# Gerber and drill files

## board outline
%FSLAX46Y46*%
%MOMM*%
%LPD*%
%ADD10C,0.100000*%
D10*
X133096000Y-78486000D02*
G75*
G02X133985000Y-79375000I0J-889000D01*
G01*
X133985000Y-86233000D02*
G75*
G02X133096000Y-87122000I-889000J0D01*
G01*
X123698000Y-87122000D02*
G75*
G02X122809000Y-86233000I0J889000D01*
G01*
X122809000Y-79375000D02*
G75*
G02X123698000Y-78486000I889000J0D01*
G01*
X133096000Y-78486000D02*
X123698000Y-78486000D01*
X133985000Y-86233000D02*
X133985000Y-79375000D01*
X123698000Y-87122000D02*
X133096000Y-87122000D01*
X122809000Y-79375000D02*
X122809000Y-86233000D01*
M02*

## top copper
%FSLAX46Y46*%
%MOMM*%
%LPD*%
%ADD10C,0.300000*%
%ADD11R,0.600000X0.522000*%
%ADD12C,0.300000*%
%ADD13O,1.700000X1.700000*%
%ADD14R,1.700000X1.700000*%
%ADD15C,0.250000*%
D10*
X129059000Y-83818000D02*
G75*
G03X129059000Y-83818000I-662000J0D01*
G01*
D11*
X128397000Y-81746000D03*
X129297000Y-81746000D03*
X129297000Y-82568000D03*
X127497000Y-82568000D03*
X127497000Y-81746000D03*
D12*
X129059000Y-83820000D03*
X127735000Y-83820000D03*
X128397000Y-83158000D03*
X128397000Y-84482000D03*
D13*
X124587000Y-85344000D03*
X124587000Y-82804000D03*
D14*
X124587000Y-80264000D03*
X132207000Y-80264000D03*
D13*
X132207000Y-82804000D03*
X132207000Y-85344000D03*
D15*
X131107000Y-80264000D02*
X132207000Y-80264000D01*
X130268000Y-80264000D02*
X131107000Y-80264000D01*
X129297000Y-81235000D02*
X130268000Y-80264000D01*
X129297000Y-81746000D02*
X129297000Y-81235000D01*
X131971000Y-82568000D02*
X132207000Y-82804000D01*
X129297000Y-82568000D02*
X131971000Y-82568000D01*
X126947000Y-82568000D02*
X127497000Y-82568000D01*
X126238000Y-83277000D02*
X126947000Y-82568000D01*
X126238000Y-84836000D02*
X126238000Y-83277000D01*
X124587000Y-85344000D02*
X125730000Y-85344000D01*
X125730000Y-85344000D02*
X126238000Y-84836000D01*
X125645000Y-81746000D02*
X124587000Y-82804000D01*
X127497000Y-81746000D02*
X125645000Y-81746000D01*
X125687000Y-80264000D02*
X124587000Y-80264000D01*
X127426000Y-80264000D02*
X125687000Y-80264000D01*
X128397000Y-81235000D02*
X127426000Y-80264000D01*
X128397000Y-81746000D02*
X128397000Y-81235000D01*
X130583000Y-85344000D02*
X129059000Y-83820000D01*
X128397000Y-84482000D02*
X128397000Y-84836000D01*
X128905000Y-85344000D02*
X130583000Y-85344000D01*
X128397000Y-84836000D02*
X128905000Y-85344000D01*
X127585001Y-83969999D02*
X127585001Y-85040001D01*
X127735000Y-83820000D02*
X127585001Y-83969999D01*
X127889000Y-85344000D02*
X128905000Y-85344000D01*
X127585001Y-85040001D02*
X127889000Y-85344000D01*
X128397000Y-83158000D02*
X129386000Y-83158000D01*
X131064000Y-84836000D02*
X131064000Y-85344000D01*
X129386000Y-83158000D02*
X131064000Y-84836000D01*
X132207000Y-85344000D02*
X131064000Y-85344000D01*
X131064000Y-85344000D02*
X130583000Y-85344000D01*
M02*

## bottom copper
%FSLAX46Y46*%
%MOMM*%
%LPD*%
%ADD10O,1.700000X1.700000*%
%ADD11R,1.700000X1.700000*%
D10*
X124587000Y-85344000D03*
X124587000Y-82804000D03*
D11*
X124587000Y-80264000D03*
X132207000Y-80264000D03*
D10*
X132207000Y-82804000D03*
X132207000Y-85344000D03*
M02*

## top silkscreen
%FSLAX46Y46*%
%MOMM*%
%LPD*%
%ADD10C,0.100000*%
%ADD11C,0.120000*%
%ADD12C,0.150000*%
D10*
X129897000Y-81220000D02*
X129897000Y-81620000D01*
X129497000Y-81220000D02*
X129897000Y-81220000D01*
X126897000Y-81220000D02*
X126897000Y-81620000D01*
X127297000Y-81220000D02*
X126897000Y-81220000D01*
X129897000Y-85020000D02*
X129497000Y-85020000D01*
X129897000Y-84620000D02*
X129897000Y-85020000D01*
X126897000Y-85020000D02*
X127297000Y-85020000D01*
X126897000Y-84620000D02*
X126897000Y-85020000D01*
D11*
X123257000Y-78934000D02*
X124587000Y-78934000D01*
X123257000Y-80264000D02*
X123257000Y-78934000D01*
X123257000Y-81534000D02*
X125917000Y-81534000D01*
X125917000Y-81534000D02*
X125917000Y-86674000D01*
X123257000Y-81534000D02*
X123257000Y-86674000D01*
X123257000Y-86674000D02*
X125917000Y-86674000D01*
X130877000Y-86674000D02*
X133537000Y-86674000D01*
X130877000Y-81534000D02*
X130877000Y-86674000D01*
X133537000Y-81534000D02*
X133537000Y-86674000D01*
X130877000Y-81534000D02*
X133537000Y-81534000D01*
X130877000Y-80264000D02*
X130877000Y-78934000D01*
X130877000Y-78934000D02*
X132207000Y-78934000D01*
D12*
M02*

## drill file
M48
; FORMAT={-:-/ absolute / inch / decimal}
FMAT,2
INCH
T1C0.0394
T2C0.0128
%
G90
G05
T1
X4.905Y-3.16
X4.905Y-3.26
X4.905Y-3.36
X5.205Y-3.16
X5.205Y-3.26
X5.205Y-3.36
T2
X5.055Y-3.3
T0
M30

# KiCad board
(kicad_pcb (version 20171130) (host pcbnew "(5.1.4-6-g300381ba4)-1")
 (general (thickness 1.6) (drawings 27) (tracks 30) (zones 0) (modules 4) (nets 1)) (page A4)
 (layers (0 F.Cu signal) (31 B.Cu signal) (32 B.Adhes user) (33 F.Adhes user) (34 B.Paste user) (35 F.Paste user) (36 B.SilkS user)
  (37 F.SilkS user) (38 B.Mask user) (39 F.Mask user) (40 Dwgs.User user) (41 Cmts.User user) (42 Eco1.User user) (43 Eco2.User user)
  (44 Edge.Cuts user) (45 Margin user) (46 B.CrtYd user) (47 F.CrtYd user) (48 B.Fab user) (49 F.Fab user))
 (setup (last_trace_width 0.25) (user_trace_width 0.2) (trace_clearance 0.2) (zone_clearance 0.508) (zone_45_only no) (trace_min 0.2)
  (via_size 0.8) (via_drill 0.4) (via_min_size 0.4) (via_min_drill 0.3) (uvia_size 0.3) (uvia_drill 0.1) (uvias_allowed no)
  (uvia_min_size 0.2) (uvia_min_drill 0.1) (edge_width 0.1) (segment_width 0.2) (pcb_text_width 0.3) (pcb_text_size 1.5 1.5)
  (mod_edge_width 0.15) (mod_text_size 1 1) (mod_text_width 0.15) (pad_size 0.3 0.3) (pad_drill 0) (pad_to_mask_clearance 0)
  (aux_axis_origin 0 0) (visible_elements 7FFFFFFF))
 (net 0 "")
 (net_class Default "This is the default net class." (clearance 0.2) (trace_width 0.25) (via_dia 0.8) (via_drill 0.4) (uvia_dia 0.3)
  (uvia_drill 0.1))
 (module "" (layer F.Cu) (at 128.397 84.48)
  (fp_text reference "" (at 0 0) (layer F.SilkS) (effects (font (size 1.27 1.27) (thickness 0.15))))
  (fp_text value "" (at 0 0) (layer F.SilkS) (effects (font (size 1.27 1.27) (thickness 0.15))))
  (fp_circle (center 0 -0.662) (end 0.662 -0.662) (layer F.Cu) (width 0.3)))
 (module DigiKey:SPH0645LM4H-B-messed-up (layer F.Cu) (at 128.397 83.82)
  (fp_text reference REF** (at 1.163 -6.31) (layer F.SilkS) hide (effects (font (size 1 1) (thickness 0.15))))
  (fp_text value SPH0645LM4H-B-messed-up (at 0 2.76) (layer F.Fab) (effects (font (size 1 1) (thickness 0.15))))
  (fp_line (start 1.5 -2.6) (end 1.5 -2.2) (layer F.SilkS) (width 0.1))
  (fp_line (start 1.1 -2.6) (end 1.5 -2.6) (layer F.SilkS) (width 0.1))
  (fp_line (start -1.5 -2.6) (end -1.5 -2.2) (layer F.SilkS) (width 0.1))
  (fp_line (start -1.1 -2.6) (end -1.5 -2.6) (layer F.SilkS) (width 0.1))
  (fp_line (start 1.5 1.2) (end 1.1 1.2) (layer F.SilkS) (width 0.1))
  (fp_line (start 1.5 0.8) (end 1.5 1.2) (layer F.SilkS) (width 0.1))
  (fp_line (start -1.5 1.2) (end -1.1 1.2) (layer F.SilkS) (width 0.1))
  (fp_line (start -1.5 0.8) (end -1.5 1.2) (layer F.SilkS) (width 0.1))
  (pad 6 smd rect (at 0 -2.074) (size 0.6 0.522) (layers F.Cu F.Paste F.Mask))
  (pad 5 smd rect (at 0.9 -2.074) (size 0.6 0.522) (layers F.Cu F.Paste F.Mask))
  (pad 4 smd rect (at 0.9 -1.252) (size 0.6 0.522) (layers F.Cu F.Paste F.Mask))
  (pad 2 smd rect (at -0.9 -1.252) (size 0.6 0.522) (layers F.Cu F.Paste F.Mask))
  (pad "" np_thru_hole circle (at 0 0) (size 0.325 0.325) (drill 0.325) (layers *.Cu *.Mask))
  (pad 1 smd rect (at -0.9 -2.074) (size 0.6 0.522) (layers F.Cu F.Paste F.Mask))
  (pad 3 smd circle (at 0.662 0) (size 0.3 0.3) (layers F.Cu F.Paste F.Mask))
  (pad 3 smd circle (at -0.662 0) (size 0.3 0.3) (layers F.Cu F.Paste F.Mask))
  (pad 3 smd circle (at 0 -0.662) (size 0.3 0.3) (layers F.Cu F.Paste F.Mask))
  (pad 3 smd circle (at 0 0.662) (size 0.3 0.3) (layers F.Cu F.Paste F.Mask)))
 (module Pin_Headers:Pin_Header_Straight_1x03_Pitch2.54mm (layer F.Cu) (at 124.587 80.264)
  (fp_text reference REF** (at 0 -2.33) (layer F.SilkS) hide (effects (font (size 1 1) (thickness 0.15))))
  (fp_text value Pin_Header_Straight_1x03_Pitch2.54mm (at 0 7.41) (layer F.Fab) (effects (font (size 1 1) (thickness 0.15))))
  (fp_line (start -1.33 -1.33) (end 0 -1.33) (layer F.SilkS) (width 0.12))
  (fp_line (start -1.33 0) (end -1.33 -1.33) (layer F.SilkS) (width 0.12))
  (fp_line (start -1.33 1.27) (end 1.33 1.27) (layer F.SilkS) (width 0.12))
  (fp_line (start 1.33 1.27) (end 1.33 6.41) (layer F.SilkS) (width 0.12))
  (fp_line (start -1.33 1.27) (end -1.33 6.41) (layer F.SilkS) (width 0.12))
  (fp_line (start -1.33 6.41) (end 1.33 6.41) (layer F.SilkS) (width 0.12))
  (pad 3 thru_hole oval (at 0 5.08) (size 1.7 1.7) (drill 1) (layers *.Cu *.Mask))
  (pad 2 thru_hole oval (at 0 2.54) (size 1.7 1.7) (drill 1) (layers *.Cu *.Mask))
  (pad 1 thru_hole rect (at 0 0) (size 1.7 1.7) (drill 1) (layers *.Cu *.Mask)))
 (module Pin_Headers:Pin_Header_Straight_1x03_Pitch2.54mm (layer F.Cu) (at 132.207 80.264)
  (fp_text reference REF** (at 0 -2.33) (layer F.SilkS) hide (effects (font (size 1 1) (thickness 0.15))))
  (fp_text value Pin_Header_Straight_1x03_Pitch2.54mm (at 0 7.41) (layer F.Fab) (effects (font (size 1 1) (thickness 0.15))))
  (fp_line (start -1.33 6.41) (end 1.33 6.41) (layer F.SilkS) (width 0.12))
  (fp_line (start -1.33 1.27) (end -1.33 6.41) (layer F.SilkS) (width 0.12))
  (fp_line (start 1.33 1.27) (end 1.33 6.41) (layer F.SilkS) (width 0.12))
  (fp_line (start -1.33 1.27) (end 1.33 1.27) (layer F.SilkS) (width 0.12))
  (fp_line (start -1.33 0) (end -1.33 -1.33) (layer F.SilkS) (width 0.12))
  (fp_line (start -1.33 -1.33) (end 0 -1.33) (layer F.SilkS) (width 0.12))
  (pad 1 thru_hole rect (at 0 0) (size 1.7 1.7) (drill 1) (layers *.Cu *.Mask))
  (pad 2 thru_hole oval (at 0 2.54) (size 1.7 1.7) (drill 1) (layers *.Cu *.Mask))
  (pad 3 thru_hole oval (at 0 5.08) (size 1.7 1.7) (drill 1) (layers *.Cu *.Mask)))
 (gr_arc (start 133.096 79.375) (end 133.985 79.375) (angle -90) (layer Edge.Cuts) (width 0.1))
 (gr_arc (start 133.096 86.233) (end 133.096 87.122) (angle -90) (layer Edge.Cuts) (width 0.1))
 (gr_arc (start 123.698 86.233) (end 122.809 86.233) (angle -90) (layer Edge.Cuts) (width 0.1))
 (gr_arc (start 123.698 79.375) (end 123.698 78.486) (angle -90) (layer Edge.Cuts) (width 0.1))
 (gr_line (start 133.096 78.486) (end 123.698 78.486) (layer Edge.Cuts) (width 0.1))
 (gr_line (start 133.985 86.233) (end 133.985 79.375) (layer Edge.Cuts) (width 0.1))
 (gr_line (start 123.698 87.122) (end 133.096 87.122) (layer Edge.Cuts) (width 0.1))
 (gr_line (start 122.809 79.375) (end 122.809 86.233) (layer Edge.Cuts) (width 0.1))
 (segment (start 131.107 80.264) (end 132.207 80.264) (width 0.25) (layer F.Cu) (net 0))
 (segment (start 130.268 80.264) (end 131.107 80.264) (width 0.25) (layer F.Cu) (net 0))
 (segment (start 129.297 81.235) (end 130.268 80.264) (width 0.25) (layer F.Cu) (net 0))
 (segment (start 129.297 81.746) (end 129.297 81.235) (width 0.25) (layer F.Cu) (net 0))
 (segment (start 131.971 82.568) (end 132.207 82.804) (width 0.25) (layer F.Cu) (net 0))
 (segment (start 129.297 82.568) (end 131.971 82.568) (width 0.25) (layer F.Cu) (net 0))
 (segment (start 126.947 82.568) (end 127.497 82.568) (width 0.25) (layer F.Cu) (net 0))
 (segment (start 126.238 83.277) (end 126.947 82.568) (width 0.25) (layer F.Cu) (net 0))
 (segment (start 126.238 84.836) (end 126.238 83.277) (width 0.25) (layer F.Cu) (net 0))
 (segment (start 124.587 85.344) (end 125.73 85.344) (width 0.25) (layer F.Cu) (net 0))
 (segment (start 125.73 85.344) (end 126.238 84.836) (width 0.25) (layer F.Cu) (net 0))
 (segment (start 125.645 81.746) (end 124.587 82.804) (width 0.25) (layer F.Cu) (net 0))
 (segment (start 127.497 81.746) (end 125.645 81.746) (width 0.25) (layer F.Cu) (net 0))
 (segment (start 125.687 80.264) (end 124.587 80.264) (width 0.25) (layer F.Cu) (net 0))
 (segment (start 127.426 80.264) (end 125.687 80.264) (width 0.25) (layer F.Cu) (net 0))
 (segment (start 128.397 81.235) (end 127.426 80.264) (width 0.25) (layer F.Cu) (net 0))
 (segment (start 128.397 81.746) (end 128.397 81.235) (width 0.25) (layer F.Cu) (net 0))
 (segment (start 130.583 85.344) (end 129.059 83.82) (width 0.25) (layer F.Cu) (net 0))
 (segment (start 128.397 84.482) (end 128.397 84.836) (width 0.25) (layer F.Cu) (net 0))
 (segment (start 128.905 85.344) (end 130.583 85.344) (width 0.25) (layer F.Cu) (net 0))
 (segment (start 128.397 84.836) (end 128.905 85.344) (width 0.25) (layer F.Cu) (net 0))
 (segment (start 127.585001 83.969999) (end 127.585001 85.040001) (width 0.25) (layer F.Cu) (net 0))
 (segment (start 127.735 83.82) (end 127.585001 83.969999) (width 0.25) (layer F.Cu) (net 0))
 (segment (start 127.889 85.344) (end 128.905 85.344) (width 0.25) (layer F.Cu) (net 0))
 (segment (start 127.585001 85.040001) (end 127.889 85.344) (width 0.25) (layer F.Cu) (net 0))
 (segment (start 128.397 83.158) (end 129.386 83.158) (width 0.25) (layer F.Cu) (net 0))
 (segment (start 131.064 84.836) (end 131.064 85.344) (width 0.25) (layer F.Cu) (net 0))
 (segment (start 129.386 83.158) (end 131.064 84.836) (width 0.25) (layer F.Cu) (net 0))
 (segment (start 132.207 85.344) (end 131.064 85.344) (width 0.25) (layer F.Cu) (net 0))
 (segment (start 131.064 85.344) (end 130.583 85.344) (width 0.25) (layer F.Cu) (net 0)))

